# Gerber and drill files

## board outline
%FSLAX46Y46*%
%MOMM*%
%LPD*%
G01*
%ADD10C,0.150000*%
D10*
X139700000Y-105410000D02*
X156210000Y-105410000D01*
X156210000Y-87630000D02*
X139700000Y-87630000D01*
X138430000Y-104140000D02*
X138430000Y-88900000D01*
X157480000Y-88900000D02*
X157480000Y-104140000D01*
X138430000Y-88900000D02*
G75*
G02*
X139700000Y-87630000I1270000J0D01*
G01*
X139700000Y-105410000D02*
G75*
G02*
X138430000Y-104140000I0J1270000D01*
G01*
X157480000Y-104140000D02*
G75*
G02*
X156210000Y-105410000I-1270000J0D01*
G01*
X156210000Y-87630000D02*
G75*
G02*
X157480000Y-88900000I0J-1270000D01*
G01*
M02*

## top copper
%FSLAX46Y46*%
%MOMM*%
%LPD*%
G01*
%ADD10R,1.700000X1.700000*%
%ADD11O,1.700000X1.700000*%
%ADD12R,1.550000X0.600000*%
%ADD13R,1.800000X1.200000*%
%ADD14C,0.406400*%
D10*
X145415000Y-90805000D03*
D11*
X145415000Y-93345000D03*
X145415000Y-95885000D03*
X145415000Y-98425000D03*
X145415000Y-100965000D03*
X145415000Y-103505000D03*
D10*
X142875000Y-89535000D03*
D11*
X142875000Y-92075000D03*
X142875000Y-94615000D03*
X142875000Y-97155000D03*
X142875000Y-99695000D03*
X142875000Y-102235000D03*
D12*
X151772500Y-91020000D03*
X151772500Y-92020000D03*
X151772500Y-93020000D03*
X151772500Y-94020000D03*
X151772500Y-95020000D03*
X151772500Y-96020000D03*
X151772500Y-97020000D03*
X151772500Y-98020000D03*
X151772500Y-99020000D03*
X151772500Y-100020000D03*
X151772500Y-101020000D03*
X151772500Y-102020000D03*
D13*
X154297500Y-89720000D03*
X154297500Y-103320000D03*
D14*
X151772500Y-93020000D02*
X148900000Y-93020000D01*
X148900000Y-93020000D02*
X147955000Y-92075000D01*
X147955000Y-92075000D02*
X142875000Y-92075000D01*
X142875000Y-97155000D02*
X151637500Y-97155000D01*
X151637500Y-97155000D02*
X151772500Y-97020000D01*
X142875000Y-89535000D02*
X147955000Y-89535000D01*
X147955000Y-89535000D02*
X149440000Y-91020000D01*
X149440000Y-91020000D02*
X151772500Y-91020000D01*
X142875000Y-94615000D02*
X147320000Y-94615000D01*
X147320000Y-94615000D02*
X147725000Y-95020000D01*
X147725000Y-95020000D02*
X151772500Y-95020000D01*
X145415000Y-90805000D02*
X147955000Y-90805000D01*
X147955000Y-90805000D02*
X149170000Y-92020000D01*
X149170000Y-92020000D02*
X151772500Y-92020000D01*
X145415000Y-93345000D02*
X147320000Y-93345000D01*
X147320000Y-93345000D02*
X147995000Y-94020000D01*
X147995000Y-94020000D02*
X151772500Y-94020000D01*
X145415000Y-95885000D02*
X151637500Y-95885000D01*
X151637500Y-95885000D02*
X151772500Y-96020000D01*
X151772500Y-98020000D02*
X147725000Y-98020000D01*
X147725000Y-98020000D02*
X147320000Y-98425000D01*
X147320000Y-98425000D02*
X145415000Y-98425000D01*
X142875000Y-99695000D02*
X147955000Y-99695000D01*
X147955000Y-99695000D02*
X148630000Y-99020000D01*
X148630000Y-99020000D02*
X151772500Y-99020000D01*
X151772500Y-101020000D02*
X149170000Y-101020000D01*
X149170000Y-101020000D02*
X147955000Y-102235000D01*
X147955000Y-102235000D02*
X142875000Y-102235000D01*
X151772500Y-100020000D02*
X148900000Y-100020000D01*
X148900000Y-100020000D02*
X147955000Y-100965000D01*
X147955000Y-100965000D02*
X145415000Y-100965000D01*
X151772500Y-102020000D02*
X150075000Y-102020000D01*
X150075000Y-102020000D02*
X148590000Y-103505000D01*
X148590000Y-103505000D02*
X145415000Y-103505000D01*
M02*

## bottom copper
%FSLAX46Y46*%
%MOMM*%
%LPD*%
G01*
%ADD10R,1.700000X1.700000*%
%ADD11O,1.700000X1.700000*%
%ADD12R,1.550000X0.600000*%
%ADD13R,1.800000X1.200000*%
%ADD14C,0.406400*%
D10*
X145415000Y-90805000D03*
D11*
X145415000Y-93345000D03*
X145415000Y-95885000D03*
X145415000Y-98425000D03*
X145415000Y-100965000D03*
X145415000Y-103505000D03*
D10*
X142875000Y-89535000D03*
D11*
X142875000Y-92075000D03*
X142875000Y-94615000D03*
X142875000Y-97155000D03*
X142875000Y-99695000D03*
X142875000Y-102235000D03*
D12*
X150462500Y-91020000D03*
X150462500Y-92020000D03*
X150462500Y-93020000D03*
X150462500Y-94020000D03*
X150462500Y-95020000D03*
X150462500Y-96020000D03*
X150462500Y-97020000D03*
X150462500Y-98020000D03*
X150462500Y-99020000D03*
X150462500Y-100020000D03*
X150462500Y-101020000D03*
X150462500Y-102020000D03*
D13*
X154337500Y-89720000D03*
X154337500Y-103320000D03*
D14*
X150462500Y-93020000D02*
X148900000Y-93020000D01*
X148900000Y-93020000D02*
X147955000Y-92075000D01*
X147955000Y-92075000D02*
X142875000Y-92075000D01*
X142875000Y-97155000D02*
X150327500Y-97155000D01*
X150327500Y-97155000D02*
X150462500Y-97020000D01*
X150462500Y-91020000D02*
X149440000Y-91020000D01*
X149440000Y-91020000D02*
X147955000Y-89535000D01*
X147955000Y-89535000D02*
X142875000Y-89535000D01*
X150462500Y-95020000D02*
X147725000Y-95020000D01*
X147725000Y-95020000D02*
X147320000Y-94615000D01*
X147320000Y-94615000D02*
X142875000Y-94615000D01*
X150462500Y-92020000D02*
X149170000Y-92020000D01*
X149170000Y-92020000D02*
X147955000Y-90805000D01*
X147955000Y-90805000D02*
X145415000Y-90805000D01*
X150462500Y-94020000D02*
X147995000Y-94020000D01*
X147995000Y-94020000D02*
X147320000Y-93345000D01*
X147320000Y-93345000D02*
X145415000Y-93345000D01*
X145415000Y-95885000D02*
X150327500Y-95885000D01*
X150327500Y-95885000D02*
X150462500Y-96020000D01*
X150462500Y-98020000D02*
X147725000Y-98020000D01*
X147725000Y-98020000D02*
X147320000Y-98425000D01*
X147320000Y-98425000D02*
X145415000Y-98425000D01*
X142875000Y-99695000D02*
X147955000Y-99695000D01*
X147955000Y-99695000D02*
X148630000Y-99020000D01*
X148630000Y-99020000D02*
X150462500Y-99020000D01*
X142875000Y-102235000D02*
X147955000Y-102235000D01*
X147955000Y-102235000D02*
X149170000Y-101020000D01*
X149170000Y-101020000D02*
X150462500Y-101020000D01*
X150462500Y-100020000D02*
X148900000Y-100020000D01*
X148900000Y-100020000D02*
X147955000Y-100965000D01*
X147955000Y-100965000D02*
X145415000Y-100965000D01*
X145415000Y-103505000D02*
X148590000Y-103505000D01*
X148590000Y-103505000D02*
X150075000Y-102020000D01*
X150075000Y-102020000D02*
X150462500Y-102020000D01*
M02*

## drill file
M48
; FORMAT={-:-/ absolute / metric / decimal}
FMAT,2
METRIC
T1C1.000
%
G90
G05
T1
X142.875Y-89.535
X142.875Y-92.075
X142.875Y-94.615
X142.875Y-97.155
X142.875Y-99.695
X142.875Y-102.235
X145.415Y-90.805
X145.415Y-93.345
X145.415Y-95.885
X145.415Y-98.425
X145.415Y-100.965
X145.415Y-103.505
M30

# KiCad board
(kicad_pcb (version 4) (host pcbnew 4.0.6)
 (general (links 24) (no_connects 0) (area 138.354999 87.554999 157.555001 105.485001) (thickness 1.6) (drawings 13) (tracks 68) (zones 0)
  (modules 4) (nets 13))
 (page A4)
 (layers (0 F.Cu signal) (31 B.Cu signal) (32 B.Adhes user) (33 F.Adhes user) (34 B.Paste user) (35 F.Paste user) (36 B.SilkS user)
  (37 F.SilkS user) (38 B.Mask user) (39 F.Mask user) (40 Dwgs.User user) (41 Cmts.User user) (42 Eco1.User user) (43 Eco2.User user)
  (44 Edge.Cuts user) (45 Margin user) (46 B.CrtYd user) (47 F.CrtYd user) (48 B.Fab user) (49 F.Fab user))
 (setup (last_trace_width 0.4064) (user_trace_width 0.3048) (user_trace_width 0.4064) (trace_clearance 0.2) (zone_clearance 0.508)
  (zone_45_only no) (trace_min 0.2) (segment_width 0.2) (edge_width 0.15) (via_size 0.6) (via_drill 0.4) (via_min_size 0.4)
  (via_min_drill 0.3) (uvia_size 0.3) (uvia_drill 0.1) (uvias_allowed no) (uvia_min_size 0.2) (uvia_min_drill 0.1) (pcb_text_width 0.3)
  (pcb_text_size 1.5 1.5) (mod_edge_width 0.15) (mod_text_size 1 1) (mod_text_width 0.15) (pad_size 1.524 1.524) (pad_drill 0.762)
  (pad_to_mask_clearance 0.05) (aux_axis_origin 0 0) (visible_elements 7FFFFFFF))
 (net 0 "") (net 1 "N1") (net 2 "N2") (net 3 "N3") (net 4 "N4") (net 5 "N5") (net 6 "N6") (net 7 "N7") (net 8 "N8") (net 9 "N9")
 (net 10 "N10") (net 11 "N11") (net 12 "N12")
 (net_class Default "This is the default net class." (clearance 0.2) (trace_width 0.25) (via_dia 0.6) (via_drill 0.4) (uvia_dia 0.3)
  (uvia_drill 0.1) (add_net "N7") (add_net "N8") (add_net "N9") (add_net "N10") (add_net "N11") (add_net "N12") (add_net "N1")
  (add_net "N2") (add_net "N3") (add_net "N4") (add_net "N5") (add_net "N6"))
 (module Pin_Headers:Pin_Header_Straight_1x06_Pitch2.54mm (layer F.Cu) (at 145.415 90.805)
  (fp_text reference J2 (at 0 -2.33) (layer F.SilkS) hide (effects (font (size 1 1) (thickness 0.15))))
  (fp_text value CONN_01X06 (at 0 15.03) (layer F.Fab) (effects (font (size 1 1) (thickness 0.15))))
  (pad 1 thru_hole rect (at 0 0) (size 1.7 1.7) (drill 1) (layers *.Cu *.Mask) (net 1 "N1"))
  (pad 2 thru_hole oval (at 0 2.54) (size 1.7 1.7) (drill 1) (layers *.Cu *.Mask) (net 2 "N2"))
  (pad 3 thru_hole oval (at 0 5.08) (size 1.7 1.7) (drill 1) (layers *.Cu *.Mask) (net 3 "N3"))
  (pad 4 thru_hole oval (at 0 7.62) (size 1.7 1.7) (drill 1) (layers *.Cu *.Mask) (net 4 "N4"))
  (pad 5 thru_hole oval (at 0 10.16) (size 1.7 1.7) (drill 1) (layers *.Cu *.Mask) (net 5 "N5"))
  (pad 6 thru_hole oval (at 0 12.7) (size 1.7 1.7) (drill 1) (layers *.Cu *.Mask) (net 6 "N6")))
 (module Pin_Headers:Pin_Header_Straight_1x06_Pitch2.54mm (layer F.Cu) (at 142.875 89.535)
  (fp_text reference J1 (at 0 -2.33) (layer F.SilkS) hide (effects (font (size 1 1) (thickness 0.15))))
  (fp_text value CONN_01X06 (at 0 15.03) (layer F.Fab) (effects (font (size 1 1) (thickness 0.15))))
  (pad 1 thru_hole rect (at 0 0) (size 1.7 1.7) (drill 1) (layers *.Cu *.Mask) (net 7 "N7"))
  (pad 2 thru_hole oval (at 0 2.54) (size 1.7 1.7) (drill 1) (layers *.Cu *.Mask) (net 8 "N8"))
  (pad 3 thru_hole oval (at 0 5.08) (size 1.7 1.7) (drill 1) (layers *.Cu *.Mask) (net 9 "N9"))
  (pad 4 thru_hole oval (at 0 7.62) (size 1.7 1.7) (drill 1) (layers *.Cu *.Mask) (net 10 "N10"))
  (pad 5 thru_hole oval (at 0 10.16) (size 1.7 1.7) (drill 1) (layers *.Cu *.Mask) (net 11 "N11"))
  (pad 6 thru_hole oval (at 0 12.7) (size 1.7 1.7) (drill 1) (layers *.Cu *.Mask) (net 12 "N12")))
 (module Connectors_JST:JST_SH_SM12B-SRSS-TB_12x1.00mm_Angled (layer B.Cu) (at 152.4 96.52 270)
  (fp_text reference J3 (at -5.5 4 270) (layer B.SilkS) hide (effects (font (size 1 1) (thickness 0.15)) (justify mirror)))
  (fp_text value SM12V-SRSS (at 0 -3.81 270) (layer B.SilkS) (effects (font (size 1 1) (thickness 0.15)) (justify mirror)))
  (pad 1 smd rect (at -5.5 1.9375 270) (size 0.6 1.55) (layers B.Cu B.Paste B.Mask) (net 7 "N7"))
  (pad 2 smd rect (at -4.5 1.9375 270) (size 0.6 1.55) (layers B.Cu B.Paste B.Mask) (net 1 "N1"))
  (pad 3 smd rect (at -3.5 1.9375 270) (size 0.6 1.55) (layers B.Cu B.Paste B.Mask) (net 8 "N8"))
  (pad 4 smd rect (at -2.5 1.9375 270) (size 0.6 1.55) (layers B.Cu B.Paste B.Mask) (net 2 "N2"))
  (pad 5 smd rect (at -1.5 1.9375 270) (size 0.6 1.55) (layers B.Cu B.Paste B.Mask) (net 9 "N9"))
  (pad 6 smd rect (at -0.5 1.9375 270) (size 0.6 1.55) (layers B.Cu B.Paste B.Mask) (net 3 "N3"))
  (pad 7 smd rect (at 0.5 1.9375 270) (size 0.6 1.55) (layers B.Cu B.Paste B.Mask) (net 10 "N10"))
  (pad 8 smd rect (at 1.5 1.9375 270) (size 0.6 1.55) (layers B.Cu B.Paste B.Mask) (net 4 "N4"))
  (pad 9 smd rect (at 2.5 1.9375 270) (size 0.6 1.55) (layers B.Cu B.Paste B.Mask) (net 11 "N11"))
  (pad 10 smd rect (at 3.5 1.9375 270) (size 0.6 1.55) (layers B.Cu B.Paste B.Mask) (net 5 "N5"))
  (pad 11 smd rect (at 4.5 1.9375 270) (size 0.6 1.55) (layers B.Cu B.Paste B.Mask) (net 12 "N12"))
  (pad 12 smd rect (at 5.5 1.9375 270) (size 0.6 1.55) (layers B.Cu B.Paste B.Mask) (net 6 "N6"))
  (pad "" smd rect (at -6.8 -1.9375 270) (size 1.2 1.8) (layers B.Cu B.Paste B.Mask))
  (pad "" smd rect (at 6.8 -1.9375 270) (size 1.2 1.8) (layers B.Cu B.Paste B.Mask)))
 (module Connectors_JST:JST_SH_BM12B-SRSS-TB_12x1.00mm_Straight (layer F.Cu) (at 153.035 96.52 270)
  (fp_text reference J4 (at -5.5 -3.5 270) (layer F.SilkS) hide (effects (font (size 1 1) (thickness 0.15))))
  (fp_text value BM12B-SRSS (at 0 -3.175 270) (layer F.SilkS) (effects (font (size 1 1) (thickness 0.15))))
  (pad 1 smd rect (at -5.5 1.2625 270) (size 0.6 1.55) (layers F.Cu F.Paste F.Mask) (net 7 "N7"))
  (pad 2 smd rect (at -4.5 1.2625 270) (size 0.6 1.55) (layers F.Cu F.Paste F.Mask) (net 1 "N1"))
  (pad 3 smd rect (at -3.5 1.2625 270) (size 0.6 1.55) (layers F.Cu F.Paste F.Mask) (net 8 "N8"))
  (pad 4 smd rect (at -2.5 1.2625 270) (size 0.6 1.55) (layers F.Cu F.Paste F.Mask) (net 2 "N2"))
  (pad 5 smd rect (at -1.5 1.2625 270) (size 0.6 1.55) (layers F.Cu F.Paste F.Mask) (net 9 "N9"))
  (pad 6 smd rect (at -0.5 1.2625 270) (size 0.6 1.55) (layers F.Cu F.Paste F.Mask) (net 3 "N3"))
  (pad 7 smd rect (at 0.5 1.2625 270) (size 0.6 1.55) (layers F.Cu F.Paste F.Mask) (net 10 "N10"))
  (pad 8 smd rect (at 1.5 1.2625 270) (size 0.6 1.55) (layers F.Cu F.Paste F.Mask) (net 4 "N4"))
  (pad 9 smd rect (at 2.5 1.2625 270) (size 0.6 1.55) (layers F.Cu F.Paste F.Mask) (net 11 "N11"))
  (pad 10 smd rect (at 3.5 1.2625 270) (size 0.6 1.55) (layers F.Cu F.Paste F.Mask) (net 5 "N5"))
  (pad 11 smd rect (at 4.5 1.2625 270) (size 0.6 1.55) (layers F.Cu F.Paste F.Mask) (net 12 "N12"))
  (pad 12 smd rect (at 5.5 1.2625 270) (size 0.6 1.55) (layers F.Cu F.Paste F.Mask) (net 6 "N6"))
  (pad "" smd rect (at -6.8 -1.2625 270) (size 1.2 1.8) (layers F.Cu F.Paste F.Mask))
  (pad "" smd rect (at 6.8 -1.2625 270) (size 1.2 1.8) (layers F.Cu F.Paste F.Mask)))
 (gr_line (start 139.7 105.41) (end 156.21 105.41) (angle 90) (layer Edge.Cuts) (width 0.15))
 (gr_line (start 156.21 87.63) (end 139.7 87.63) (angle 90) (layer Edge.Cuts) (width 0.15))
 (gr_line (start 138.43 104.14) (end 138.43 88.9) (angle 90) (layer Edge.Cuts) (width 0.15))
 (gr_line (start 157.48 88.9) (end 157.48 104.14) (angle 90) (layer Edge.Cuts) (width 0.15))
 (gr_arc (start 139.7 88.9) (end 138.43 88.9) (angle 90) (layer Edge.Cuts) (width 0.15))
 (gr_arc (start 139.7 104.14) (end 139.7 105.41) (angle 90) (layer Edge.Cuts) (width 0.15))
 (gr_arc (start 156.21 104.14) (end 157.48 104.14) (angle 90) (layer Edge.Cuts) (width 0.15))
 (gr_arc (start 156.21 88.9) (end 156.21 87.63) (angle 90) (layer Edge.Cuts) (width 0.15))
 (segment (start 150.4625 93.02) (end 148.9 93.02) (width 0.4064) (layer B.Cu) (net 8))
 (segment (start 148.9 93.02) (end 147.955 92.075) (width 0.4064) (layer B.Cu) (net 8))
 (segment (start 147.955 92.075) (end 142.875 92.075) (width 0.4064) (layer B.Cu) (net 8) (status 20))
 (segment (start 151.7725 93.02) (end 148.9 93.02) (width 0.4064) (layer F.Cu) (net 8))
 (segment (start 148.9 93.02) (end 147.955 92.075) (width 0.4064) (layer F.Cu) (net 8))
 (segment (start 147.955 92.075) (end 142.875 92.075) (width 0.4064) (layer F.Cu) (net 8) (status 20))
 (segment (start 142.875 97.155) (end 150.3275 97.155) (width 0.4064) (layer B.Cu) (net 10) (status 10))
 (segment (start 150.3275 97.155) (end 150.4625 97.02) (width 0.4064) (layer B.Cu) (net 10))
 (segment (start 142.875 97.155) (end 151.6375 97.155) (width 0.4064) (layer F.Cu) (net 10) (status 10))
 (segment (start 151.6375 97.155) (end 151.7725 97.02) (width 0.4064) (layer F.Cu) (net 10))
 (segment (start 150.4625 91.02) (end 149.44 91.02) (width 0.4064) (layer B.Cu) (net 7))
 (segment (start 149.44 91.02) (end 147.955 89.535) (width 0.4064) (layer B.Cu) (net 7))
 (segment (start 147.955 89.535) (end 142.875 89.535) (width 0.4064) (layer B.Cu) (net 7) (status 20))
 (segment (start 142.875 89.535) (end 147.955 89.535) (width 0.4064) (layer F.Cu) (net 7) (status 10))
 (segment (start 147.955 89.535) (end 149.44 91.02) (width 0.4064) (layer F.Cu) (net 7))
 (segment (start 149.44 91.02) (end 151.7725 91.02) (width 0.4064) (layer F.Cu) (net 7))
 (segment (start 150.4625 95.02) (end 147.725 95.02) (width 0.4064) (layer B.Cu) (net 9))
 (segment (start 147.725 95.02) (end 147.32 94.615) (width 0.4064) (layer B.Cu) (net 9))
 (segment (start 147.32 94.615) (end 142.875 94.615) (width 0.4064) (layer B.Cu) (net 9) (status 20))
 (segment (start 142.875 94.615) (end 147.32 94.615) (width 0.4064) (layer F.Cu) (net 9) (status 10))
 (segment (start 147.32 94.615) (end 147.725 95.02) (width 0.4064) (layer F.Cu) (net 9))
 (segment (start 147.725 95.02) (end 151.7725 95.02) (width 0.4064) (layer F.Cu) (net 9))
 (segment (start 150.4625 92.02) (end 149.17 92.02) (width 0.4064) (layer B.Cu) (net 1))
 (segment (start 149.17 92.02) (end 147.955 90.805) (width 0.4064) (layer B.Cu) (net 1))
 (segment (start 147.955 90.805) (end 145.415 90.805) (width 0.4064) (layer B.Cu) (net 1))
 (segment (start 145.415 90.805) (end 147.955 90.805) (width 0.4064) (layer F.Cu) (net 1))
 (segment (start 147.955 90.805) (end 149.17 92.02) (width 0.4064) (layer F.Cu) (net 1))
 (segment (start 149.17 92.02) (end 151.7725 92.02) (width 0.4064) (layer F.Cu) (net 1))
 (segment (start 150.4625 94.02) (end 147.995 94.02) (width 0.4064) (layer B.Cu) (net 2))
 (segment (start 147.995 94.02) (end 147.32 93.345) (width 0.4064) (layer B.Cu) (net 2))
 (segment (start 147.32 93.345) (end 145.415 93.345) (width 0.4064) (layer B.Cu) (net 2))
 (segment (start 145.415 93.345) (end 147.32 93.345) (width 0.4064) (layer F.Cu) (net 2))
 (segment (start 147.32 93.345) (end 147.995 94.02) (width 0.4064) (layer F.Cu) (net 2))
 (segment (start 147.995 94.02) (end 151.7725 94.02) (width 0.4064) (layer F.Cu) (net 2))
 (segment (start 145.415 95.885) (end 150.3275 95.885) (width 0.4064) (layer B.Cu) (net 3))
 (segment (start 150.3275 95.885) (end 150.4625 96.02) (width 0.4064) (layer B.Cu) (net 3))
 (segment (start 145.415 95.885) (end 151.6375 95.885) (width 0.4064) (layer F.Cu) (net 3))
 (segment (start 151.6375 95.885) (end 151.7725 96.02) (width 0.4064) (layer F.Cu) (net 3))
 (segment (start 150.4625 98.02) (end 147.725 98.02) (width 0.4064) (layer B.Cu) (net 4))
 (segment (start 147.725 98.02) (end 147.32 98.425) (width 0.4064) (layer B.Cu) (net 4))
 (segment (start 147.32 98.425) (end 145.415 98.425) (width 0.4064) (layer B.Cu) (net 4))
 (segment (start 151.7725 98.02) (end 147.725 98.02) (width 0.4064) (layer F.Cu) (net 4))
 (segment (start 147.725 98.02) (end 147.32 98.425) (width 0.4064) (layer F.Cu) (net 4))
 (segment (start 147.32 98.425) (end 145.415 98.425) (width 0.4064) (layer F.Cu) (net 4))
 (segment (start 142.875 99.695) (end 147.955 99.695) (width 0.4064) (layer B.Cu) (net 11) (status 10))
 (segment (start 147.955 99.695) (end 148.63 99.02) (width 0.4064) (layer B.Cu) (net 11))
 (segment (start 148.63 99.02) (end 150.4625 99.02) (width 0.4064) (layer B.Cu) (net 11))
 (segment (start 142.875 99.695) (end 147.955 99.695) (width 0.4064) (layer F.Cu) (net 11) (status 10))
 (segment (start 147.955 99.695) (end 148.63 99.02) (width 0.4064) (layer F.Cu) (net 11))
 (segment (start 148.63 99.02) (end 151.7725 99.02) (width 0.4064) (layer F.Cu) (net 11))
 (segment (start 142.875 102.235) (end 147.955 102.235) (width 0.4064) (layer B.Cu) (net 12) (status 10))
 (segment (start 147.955 102.235) (end 149.17 101.02) (width 0.4064) (layer B.Cu) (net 12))
 (segment (start 149.17 101.02) (end 150.4625 101.02) (width 0.4064) (layer B.Cu) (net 12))
 (segment (start 151.7725 101.02) (end 149.17 101.02) (width 0.4064) (layer F.Cu) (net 12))
 (segment (start 149.17 101.02) (end 147.955 102.235) (width 0.4064) (layer F.Cu) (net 12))
 (segment (start 147.955 102.235) (end 142.875 102.235) (width 0.4064) (layer F.Cu) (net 12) (status 20))
 (segment (start 150.4625 100.02) (end 148.9 100.02) (width 0.4064) (layer B.Cu) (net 5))
 (segment (start 148.9 100.02) (end 147.955 100.965) (width 0.4064) (layer B.Cu) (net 5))
 (segment (start 147.955 100.965) (end 145.415 100.965) (width 0.4064) (layer B.Cu) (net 5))
 (segment (start 151.7725 100.02) (end 148.9 100.02) (width 0.4064) (layer F.Cu) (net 5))
 (segment (start 148.9 100.02) (end 147.955 100.965) (width 0.4064) (layer F.Cu) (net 5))
 (segment (start 147.955 100.965) (end 145.415 100.965) (width 0.4064) (layer F.Cu) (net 5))
 (segment (start 145.415 103.505) (end 148.59 103.505) (width 0.4064) (layer B.Cu) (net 6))
 (segment (start 148.59 103.505) (end 150.075 102.02) (width 0.4064) (layer B.Cu) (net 6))
 (segment (start 150.075 102.02) (end 150.4625 102.02) (width 0.4064) (layer B.Cu) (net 6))
 (segment (start 151.7725 102.02) (end 150.075 102.02) (width 0.4064) (layer F.Cu) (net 6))
 (segment (start 150.075 102.02) (end 148.59 103.505) (width 0.4064) (layer F.Cu) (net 6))
 (segment (start 148.59 103.505) (end 145.415 103.505) (width 0.4064) (layer F.Cu) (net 6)))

